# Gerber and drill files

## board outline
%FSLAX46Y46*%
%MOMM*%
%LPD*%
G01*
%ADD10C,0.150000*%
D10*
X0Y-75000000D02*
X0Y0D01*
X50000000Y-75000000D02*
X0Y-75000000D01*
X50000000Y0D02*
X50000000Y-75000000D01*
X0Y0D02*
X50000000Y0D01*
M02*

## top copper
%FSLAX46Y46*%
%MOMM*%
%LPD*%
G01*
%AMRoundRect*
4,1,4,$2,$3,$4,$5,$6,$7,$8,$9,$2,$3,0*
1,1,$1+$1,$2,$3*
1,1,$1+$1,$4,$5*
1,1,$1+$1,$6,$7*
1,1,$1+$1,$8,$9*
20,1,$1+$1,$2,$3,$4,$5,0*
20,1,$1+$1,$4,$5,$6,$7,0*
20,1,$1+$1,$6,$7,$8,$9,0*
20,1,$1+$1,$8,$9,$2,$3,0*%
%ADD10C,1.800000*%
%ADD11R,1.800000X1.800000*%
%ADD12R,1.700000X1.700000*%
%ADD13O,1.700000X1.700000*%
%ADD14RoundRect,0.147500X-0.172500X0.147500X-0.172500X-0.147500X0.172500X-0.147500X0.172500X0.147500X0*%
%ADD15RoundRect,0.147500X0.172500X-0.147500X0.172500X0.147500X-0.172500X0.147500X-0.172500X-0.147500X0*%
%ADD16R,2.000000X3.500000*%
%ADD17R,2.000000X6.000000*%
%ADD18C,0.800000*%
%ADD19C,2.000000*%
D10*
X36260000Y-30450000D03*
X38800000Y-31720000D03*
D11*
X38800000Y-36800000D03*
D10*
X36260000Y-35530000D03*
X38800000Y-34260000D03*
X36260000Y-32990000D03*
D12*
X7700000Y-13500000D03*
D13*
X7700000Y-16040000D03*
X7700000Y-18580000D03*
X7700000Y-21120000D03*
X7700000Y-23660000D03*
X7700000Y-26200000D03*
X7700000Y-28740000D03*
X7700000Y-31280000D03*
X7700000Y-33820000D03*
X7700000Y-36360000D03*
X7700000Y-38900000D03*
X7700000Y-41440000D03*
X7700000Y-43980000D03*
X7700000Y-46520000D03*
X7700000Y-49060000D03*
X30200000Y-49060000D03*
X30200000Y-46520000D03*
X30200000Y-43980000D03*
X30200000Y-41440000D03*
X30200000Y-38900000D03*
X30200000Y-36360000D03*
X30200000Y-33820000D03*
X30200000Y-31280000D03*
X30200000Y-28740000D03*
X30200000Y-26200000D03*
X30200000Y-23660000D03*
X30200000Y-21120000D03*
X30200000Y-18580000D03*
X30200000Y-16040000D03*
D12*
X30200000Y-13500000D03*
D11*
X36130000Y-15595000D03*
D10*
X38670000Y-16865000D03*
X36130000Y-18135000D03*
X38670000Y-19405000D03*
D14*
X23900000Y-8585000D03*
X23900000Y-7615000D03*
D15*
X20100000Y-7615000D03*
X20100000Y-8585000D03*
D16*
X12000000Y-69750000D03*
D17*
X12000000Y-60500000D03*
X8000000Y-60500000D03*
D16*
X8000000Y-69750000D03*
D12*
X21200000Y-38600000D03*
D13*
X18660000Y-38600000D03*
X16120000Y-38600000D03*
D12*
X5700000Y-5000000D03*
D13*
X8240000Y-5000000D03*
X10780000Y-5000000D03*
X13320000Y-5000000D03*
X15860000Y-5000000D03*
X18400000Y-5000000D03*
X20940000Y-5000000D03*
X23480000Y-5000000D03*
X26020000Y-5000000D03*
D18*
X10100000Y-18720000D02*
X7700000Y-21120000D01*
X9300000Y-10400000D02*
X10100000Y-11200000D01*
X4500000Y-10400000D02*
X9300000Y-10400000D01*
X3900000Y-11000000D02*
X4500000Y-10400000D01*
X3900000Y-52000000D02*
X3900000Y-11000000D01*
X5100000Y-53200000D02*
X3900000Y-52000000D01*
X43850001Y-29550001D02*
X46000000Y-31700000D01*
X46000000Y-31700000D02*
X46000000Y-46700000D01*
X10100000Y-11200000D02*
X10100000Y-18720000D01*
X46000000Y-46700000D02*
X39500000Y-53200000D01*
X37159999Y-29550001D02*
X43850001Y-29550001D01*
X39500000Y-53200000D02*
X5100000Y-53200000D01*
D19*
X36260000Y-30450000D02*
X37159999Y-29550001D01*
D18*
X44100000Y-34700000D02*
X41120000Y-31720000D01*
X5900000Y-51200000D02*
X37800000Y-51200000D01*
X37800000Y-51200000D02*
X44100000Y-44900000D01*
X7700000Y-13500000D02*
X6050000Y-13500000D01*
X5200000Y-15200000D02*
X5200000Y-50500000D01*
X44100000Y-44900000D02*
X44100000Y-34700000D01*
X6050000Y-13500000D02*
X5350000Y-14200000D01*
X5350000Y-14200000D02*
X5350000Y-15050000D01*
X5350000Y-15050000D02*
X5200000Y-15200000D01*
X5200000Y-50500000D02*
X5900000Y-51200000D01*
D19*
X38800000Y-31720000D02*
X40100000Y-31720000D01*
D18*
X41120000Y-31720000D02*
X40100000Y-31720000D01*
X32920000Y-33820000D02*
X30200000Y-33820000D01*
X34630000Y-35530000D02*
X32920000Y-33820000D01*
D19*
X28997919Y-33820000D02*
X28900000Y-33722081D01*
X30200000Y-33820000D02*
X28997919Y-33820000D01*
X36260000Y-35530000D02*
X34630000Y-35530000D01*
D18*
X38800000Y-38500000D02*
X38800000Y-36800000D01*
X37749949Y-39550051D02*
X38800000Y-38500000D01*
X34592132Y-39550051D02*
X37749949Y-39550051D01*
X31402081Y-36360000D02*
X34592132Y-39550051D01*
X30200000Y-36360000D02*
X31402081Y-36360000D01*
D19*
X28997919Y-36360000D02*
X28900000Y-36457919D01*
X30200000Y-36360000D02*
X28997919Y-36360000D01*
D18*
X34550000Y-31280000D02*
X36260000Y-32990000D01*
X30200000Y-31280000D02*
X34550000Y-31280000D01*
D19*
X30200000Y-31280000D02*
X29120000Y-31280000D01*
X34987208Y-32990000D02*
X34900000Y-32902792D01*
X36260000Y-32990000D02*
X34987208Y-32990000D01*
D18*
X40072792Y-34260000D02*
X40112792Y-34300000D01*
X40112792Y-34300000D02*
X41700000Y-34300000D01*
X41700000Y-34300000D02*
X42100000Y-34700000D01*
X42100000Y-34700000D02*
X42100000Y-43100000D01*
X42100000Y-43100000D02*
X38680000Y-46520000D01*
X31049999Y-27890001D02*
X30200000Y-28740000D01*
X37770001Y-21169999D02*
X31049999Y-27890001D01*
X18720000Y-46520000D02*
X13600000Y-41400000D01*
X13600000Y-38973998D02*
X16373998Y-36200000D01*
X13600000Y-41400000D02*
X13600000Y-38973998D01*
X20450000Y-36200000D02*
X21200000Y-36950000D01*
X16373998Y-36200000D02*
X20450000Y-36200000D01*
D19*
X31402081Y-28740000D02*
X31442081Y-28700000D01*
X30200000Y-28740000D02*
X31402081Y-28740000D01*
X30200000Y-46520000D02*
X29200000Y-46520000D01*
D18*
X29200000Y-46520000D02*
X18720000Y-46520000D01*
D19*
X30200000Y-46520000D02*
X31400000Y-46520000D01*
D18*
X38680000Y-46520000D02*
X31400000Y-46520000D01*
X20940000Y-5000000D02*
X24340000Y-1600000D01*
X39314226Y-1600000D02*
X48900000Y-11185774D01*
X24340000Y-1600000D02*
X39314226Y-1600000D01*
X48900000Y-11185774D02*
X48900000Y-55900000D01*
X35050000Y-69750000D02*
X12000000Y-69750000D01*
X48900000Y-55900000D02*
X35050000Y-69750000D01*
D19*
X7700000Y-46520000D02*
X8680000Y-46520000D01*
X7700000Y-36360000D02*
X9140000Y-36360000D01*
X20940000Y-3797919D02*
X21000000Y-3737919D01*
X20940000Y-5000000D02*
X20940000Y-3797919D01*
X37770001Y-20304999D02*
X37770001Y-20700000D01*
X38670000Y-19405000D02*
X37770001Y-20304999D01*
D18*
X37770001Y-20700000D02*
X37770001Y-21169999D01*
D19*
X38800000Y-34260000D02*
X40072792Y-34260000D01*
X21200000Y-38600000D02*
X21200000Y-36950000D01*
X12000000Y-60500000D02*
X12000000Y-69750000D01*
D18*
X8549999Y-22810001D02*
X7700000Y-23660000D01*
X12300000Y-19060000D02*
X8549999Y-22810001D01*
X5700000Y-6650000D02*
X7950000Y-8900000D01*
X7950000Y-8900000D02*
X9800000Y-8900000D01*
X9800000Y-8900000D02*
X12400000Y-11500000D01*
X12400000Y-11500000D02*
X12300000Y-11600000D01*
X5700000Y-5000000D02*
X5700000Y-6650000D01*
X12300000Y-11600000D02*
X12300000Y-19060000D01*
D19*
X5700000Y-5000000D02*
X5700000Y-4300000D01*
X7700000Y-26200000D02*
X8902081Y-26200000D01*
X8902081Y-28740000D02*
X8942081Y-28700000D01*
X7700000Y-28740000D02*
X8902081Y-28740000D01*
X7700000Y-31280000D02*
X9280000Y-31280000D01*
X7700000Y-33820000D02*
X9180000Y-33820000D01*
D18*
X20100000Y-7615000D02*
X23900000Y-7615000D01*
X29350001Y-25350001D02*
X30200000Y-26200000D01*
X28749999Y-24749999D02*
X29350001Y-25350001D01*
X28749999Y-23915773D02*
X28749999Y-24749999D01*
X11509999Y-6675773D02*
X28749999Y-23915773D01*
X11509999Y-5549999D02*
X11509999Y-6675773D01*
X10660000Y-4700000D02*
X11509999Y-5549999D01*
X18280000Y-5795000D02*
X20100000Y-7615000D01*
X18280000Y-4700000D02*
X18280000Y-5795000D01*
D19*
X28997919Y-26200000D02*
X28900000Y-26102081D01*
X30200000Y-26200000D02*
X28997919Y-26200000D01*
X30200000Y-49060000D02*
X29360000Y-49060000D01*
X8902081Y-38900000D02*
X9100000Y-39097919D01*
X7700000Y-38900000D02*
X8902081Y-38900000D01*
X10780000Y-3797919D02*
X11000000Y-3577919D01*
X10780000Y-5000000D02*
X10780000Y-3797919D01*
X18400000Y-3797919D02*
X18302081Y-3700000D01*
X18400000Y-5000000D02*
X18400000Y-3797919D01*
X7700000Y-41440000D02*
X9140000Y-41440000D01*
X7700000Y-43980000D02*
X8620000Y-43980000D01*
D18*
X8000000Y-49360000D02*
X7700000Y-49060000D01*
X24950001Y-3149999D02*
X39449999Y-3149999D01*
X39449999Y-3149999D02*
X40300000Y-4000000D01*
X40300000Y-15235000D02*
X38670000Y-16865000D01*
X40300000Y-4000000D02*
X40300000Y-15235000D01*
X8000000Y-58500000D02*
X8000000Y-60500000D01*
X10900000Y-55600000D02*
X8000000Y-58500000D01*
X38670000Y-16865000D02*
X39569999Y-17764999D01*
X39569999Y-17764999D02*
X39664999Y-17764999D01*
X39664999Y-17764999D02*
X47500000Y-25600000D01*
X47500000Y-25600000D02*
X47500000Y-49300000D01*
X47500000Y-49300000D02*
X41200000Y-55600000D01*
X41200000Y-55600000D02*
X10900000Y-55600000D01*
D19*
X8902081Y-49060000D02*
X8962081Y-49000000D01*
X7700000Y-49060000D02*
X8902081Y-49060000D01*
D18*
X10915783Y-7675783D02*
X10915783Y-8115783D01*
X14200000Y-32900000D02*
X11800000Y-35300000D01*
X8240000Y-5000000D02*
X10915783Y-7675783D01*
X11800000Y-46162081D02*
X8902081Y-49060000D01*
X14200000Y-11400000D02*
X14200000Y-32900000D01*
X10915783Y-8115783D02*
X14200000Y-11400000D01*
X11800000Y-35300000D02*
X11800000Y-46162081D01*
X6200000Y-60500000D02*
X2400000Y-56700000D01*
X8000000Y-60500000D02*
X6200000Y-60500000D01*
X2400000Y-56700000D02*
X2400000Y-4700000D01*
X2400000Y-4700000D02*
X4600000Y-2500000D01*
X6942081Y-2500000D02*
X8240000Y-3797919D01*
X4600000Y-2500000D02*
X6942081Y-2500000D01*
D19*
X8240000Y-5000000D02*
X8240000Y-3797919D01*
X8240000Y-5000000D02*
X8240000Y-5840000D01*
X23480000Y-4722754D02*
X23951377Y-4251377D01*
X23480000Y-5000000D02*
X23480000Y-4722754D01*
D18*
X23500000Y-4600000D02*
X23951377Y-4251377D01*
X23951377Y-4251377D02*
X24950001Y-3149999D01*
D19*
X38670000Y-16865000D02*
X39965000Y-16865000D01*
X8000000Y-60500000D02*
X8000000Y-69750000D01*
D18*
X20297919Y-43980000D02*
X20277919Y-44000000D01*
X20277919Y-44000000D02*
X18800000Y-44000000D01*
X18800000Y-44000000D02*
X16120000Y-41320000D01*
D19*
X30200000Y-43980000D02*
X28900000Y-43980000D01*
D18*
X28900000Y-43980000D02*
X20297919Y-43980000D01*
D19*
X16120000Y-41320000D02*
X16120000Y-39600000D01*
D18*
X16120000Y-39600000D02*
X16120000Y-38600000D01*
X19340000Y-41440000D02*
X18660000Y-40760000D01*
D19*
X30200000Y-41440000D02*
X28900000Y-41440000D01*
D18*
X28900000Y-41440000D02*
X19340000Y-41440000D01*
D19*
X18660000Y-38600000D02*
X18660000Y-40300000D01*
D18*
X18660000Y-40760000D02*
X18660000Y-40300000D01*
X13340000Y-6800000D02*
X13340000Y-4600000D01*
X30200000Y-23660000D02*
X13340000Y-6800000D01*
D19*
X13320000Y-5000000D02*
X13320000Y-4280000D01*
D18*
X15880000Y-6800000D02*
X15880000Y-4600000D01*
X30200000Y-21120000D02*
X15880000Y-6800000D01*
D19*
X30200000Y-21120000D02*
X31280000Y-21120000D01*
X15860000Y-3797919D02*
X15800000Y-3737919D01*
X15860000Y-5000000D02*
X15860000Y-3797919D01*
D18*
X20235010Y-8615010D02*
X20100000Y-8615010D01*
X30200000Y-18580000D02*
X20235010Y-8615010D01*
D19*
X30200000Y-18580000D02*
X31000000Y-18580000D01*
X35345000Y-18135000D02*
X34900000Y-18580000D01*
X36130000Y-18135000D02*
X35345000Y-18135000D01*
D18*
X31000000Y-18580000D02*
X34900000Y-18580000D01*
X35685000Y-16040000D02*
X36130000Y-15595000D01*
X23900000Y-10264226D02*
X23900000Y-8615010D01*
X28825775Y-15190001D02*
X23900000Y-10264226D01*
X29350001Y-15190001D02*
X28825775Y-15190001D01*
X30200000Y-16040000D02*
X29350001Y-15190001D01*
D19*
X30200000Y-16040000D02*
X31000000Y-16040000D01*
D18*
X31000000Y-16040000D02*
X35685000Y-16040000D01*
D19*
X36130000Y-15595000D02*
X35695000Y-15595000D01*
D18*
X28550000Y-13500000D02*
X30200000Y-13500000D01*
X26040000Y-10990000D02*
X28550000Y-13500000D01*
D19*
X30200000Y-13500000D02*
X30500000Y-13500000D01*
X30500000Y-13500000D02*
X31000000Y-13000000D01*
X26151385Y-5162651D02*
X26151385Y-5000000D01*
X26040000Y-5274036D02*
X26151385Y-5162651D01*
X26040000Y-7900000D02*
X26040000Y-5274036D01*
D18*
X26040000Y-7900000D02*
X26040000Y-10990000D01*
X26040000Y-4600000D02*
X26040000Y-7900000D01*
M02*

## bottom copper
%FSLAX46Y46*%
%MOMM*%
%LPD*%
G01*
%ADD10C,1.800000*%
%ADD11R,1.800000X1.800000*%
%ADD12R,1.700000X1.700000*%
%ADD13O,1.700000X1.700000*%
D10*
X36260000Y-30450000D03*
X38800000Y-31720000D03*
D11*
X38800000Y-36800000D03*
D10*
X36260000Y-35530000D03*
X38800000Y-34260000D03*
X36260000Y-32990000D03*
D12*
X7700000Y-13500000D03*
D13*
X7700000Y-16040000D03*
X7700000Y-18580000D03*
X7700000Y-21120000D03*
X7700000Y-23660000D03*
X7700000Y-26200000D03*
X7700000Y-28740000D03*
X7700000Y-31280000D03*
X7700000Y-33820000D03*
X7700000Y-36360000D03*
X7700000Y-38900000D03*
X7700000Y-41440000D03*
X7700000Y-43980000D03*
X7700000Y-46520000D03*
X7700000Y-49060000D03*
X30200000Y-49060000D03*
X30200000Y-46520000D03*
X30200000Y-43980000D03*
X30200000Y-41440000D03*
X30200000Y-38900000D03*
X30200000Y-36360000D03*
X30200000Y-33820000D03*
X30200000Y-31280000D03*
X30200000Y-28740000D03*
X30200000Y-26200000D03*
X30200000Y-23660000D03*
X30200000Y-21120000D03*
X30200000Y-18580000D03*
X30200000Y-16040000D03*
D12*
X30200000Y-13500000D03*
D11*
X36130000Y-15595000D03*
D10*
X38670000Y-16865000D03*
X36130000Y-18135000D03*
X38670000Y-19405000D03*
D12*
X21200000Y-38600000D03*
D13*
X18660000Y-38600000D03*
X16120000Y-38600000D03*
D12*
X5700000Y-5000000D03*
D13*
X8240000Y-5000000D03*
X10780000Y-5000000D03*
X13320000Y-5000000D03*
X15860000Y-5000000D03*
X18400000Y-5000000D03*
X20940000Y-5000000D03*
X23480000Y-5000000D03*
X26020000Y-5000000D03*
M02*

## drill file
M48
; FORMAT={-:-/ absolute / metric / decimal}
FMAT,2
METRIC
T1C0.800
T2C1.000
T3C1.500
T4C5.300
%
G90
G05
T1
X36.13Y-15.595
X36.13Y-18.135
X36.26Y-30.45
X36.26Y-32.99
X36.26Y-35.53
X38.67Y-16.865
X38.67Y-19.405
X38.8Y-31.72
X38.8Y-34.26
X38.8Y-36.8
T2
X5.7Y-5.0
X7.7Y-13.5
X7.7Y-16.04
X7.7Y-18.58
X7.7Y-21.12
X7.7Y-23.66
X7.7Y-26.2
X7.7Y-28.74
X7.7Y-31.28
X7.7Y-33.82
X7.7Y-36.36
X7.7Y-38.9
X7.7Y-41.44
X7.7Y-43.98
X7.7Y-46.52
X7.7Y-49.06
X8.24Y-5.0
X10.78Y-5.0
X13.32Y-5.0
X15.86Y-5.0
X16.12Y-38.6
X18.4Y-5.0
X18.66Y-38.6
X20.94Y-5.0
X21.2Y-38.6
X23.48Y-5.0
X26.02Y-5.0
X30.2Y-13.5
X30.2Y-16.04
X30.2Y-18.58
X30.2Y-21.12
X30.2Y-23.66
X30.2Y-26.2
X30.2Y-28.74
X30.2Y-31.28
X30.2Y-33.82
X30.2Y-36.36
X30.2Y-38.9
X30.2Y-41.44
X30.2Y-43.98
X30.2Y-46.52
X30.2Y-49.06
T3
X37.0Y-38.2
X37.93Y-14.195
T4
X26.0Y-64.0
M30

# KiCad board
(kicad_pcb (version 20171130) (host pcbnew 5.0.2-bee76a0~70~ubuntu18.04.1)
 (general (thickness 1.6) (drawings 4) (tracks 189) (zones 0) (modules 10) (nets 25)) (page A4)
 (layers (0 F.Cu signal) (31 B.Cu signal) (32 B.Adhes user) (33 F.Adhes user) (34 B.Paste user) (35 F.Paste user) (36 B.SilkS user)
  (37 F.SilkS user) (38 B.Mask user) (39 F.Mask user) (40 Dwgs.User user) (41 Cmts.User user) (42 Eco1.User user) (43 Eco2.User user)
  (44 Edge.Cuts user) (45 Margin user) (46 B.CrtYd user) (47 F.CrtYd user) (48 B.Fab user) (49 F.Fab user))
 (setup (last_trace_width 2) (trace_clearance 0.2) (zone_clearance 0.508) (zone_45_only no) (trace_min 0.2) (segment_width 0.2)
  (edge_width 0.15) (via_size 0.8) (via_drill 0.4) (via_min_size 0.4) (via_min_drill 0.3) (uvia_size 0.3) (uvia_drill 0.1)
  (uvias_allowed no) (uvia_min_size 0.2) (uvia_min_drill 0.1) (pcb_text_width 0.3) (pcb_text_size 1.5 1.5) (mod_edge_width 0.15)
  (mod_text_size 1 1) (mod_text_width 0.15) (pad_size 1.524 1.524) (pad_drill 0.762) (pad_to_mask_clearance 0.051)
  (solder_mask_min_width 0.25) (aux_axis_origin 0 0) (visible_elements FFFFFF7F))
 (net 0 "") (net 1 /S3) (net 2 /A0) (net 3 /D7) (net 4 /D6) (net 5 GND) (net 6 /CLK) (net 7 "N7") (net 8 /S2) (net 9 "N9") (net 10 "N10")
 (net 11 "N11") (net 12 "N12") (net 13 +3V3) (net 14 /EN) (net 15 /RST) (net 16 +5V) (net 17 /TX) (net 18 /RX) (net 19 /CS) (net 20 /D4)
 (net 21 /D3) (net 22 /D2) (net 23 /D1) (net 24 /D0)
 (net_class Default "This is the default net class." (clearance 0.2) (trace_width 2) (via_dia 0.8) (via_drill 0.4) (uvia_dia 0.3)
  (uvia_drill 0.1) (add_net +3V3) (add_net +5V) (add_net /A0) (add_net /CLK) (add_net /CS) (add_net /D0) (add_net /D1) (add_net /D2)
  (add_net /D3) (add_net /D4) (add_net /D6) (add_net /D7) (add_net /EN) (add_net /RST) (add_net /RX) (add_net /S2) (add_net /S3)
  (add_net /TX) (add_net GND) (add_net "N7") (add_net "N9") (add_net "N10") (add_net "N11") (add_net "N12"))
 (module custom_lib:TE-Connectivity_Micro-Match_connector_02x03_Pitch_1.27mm (layer F.Cu) (at 38.8 36.8 180)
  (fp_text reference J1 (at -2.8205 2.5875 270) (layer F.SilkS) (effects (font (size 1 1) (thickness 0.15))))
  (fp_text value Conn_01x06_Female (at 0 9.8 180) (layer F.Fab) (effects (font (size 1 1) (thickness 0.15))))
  (pad 6 thru_hole circle (at 2.54 6.35 180) (size 1.8 1.8) (drill 0.8001) (layers *.Cu *.Mask) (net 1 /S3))
  (pad 5 thru_hole circle (at 0 5.08 180) (size 1.8 1.8) (drill 0.8001) (layers *.Cu *.Mask) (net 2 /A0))
  (pad 1 thru_hole rect (at 0 0 180) (size 1.8 1.8) (drill 0.8001) (layers *.Cu *.Mask) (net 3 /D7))
  (pad 2 thru_hole circle (at 2.54 1.27 180) (size 1.8 1.8) (drill 0.8001) (layers *.Cu *.Mask) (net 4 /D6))
  (pad 3 thru_hole circle (at 0 2.54 180) (size 1.8 1.8) (drill 0.8001) (layers *.Cu *.Mask) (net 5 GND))
  (pad 4 thru_hole circle (at 2.54 3.81 180) (size 1.8 1.8) (drill 0.8001) (layers *.Cu *.Mask) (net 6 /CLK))
  (pad "" np_thru_hole circle (at 1.8 -1.4 180) (size 1.5001 1.5001) (drill 1.5001) (layers *.Cu *.Mask)))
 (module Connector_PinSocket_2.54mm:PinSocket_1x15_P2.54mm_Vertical (layer F.Cu) (at 7.7 13.5)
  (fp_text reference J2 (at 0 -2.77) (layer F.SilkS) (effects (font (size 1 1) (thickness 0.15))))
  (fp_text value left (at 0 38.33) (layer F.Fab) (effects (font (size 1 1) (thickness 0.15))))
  (pad 1 thru_hole rect (at 0 0) (size 1.7 1.7) (drill 1) (layers *.Cu *.Mask) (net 2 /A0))
  (pad 2 thru_hole oval (at 0 2.54) (size 1.7 1.7) (drill 1) (layers *.Cu *.Mask) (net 5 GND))
  (pad 3 thru_hole oval (at 0 5.08) (size 1.7 1.7) (drill 1) (layers *.Cu *.Mask) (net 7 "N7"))
  (pad 4 thru_hole oval (at 0 7.62) (size 1.7 1.7) (drill 1) (layers *.Cu *.Mask) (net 1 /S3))
  (pad 5 thru_hole oval (at 0 10.16) (size 1.7 1.7) (drill 1) (layers *.Cu *.Mask) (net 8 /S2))
  (pad 6 thru_hole oval (at 0 12.7) (size 1.7 1.7) (drill 1) (layers *.Cu *.Mask) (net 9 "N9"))
  (pad 7 thru_hole oval (at 0 15.24) (size 1.7 1.7) (drill 1) (layers *.Cu *.Mask) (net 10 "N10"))
  (pad 8 thru_hole oval (at 0 17.78) (size 1.7 1.7) (drill 1) (layers *.Cu *.Mask) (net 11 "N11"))
  (pad 9 thru_hole oval (at 0 20.32) (size 1.7 1.7) (drill 1) (layers *.Cu *.Mask) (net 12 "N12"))
  (pad 10 thru_hole oval (at 0 22.86) (size 1.7 1.7) (drill 1) (layers *.Cu *.Mask) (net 5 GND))
  (pad 11 thru_hole oval (at 0 25.4) (size 1.7 1.7) (drill 1) (layers *.Cu *.Mask) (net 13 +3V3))
  (pad 12 thru_hole oval (at 0 27.94) (size 1.7 1.7) (drill 1) (layers *.Cu *.Mask) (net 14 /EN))
  (pad 13 thru_hole oval (at 0 30.48) (size 1.7 1.7) (drill 1) (layers *.Cu *.Mask) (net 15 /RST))
  (pad 14 thru_hole oval (at 0 33.02) (size 1.7 1.7) (drill 1) (layers *.Cu *.Mask) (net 5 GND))
  (pad 15 thru_hole oval (at 0 35.56) (size 1.7 1.7) (drill 1) (layers *.Cu *.Mask) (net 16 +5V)))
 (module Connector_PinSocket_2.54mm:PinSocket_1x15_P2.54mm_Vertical (layer F.Cu) (at 30.2 13.5)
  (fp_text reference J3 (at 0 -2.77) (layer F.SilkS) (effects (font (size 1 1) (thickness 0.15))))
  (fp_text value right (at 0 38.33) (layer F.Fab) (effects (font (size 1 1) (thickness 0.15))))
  (pad 15 thru_hole oval (at 0 35.56) (size 1.7 1.7) (drill 1) (layers *.Cu *.Mask) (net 13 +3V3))
  (pad 14 thru_hole oval (at 0 33.02) (size 1.7 1.7) (drill 1) (layers *.Cu *.Mask) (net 5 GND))
  (pad 13 thru_hole oval (at 0 30.48) (size 1.7 1.7) (drill 1) (layers *.Cu *.Mask) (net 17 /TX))
  (pad 12 thru_hole oval (at 0 27.94) (size 1.7 1.7) (drill 1) (layers *.Cu *.Mask) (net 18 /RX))
  (pad 11 thru_hole oval (at 0 25.4) (size 1.7 1.7) (drill 1) (layers *.Cu *.Mask) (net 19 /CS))
  (pad 10 thru_hole oval (at 0 22.86) (size 1.7 1.7) (drill 1) (layers *.Cu *.Mask) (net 3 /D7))
  (pad 9 thru_hole oval (at 0 20.32) (size 1.7 1.7) (drill 1) (layers *.Cu *.Mask) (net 4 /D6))
  (pad 8 thru_hole oval (at 0 17.78) (size 1.7 1.7) (drill 1) (layers *.Cu *.Mask) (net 6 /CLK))
  (pad 7 thru_hole oval (at 0 15.24) (size 1.7 1.7) (drill 1) (layers *.Cu *.Mask) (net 5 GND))
  (pad 6 thru_hole oval (at 0 12.7) (size 1.7 1.7) (drill 1) (layers *.Cu *.Mask) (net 13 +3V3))
  (pad 5 thru_hole oval (at 0 10.16) (size 1.7 1.7) (drill 1) (layers *.Cu *.Mask) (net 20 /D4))
  (pad 4 thru_hole oval (at 0 7.62) (size 1.7 1.7) (drill 1) (layers *.Cu *.Mask) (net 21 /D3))
  (pad 3 thru_hole oval (at 0 5.08) (size 1.7 1.7) (drill 1) (layers *.Cu *.Mask) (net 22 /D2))
  (pad 2 thru_hole oval (at 0 2.54) (size 1.7 1.7) (drill 1) (layers *.Cu *.Mask) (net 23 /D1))
  (pad 1 thru_hole rect (at 0 0) (size 1.7 1.7) (drill 1) (layers *.Cu *.Mask) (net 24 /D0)))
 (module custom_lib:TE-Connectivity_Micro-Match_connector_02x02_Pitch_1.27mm (layer F.Cu) (at 37.4 17.5)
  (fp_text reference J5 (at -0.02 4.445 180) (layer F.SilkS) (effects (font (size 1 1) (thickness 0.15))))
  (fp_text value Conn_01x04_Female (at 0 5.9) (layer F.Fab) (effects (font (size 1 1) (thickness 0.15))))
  (pad 1 thru_hole rect (at -1.27 -1.905) (size 1.8 1.8) (drill 0.8001) (layers *.Cu *.Mask) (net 23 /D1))
  (pad 2 thru_hole circle (at 1.27 -0.635) (size 1.8 1.8) (drill 0.8001) (layers *.Cu *.Mask) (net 16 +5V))
  (pad 3 thru_hole circle (at -1.27 0.635) (size 1.8 1.8) (drill 0.8001) (layers *.Cu *.Mask) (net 22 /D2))
  (pad 4 thru_hole circle (at 1.27 1.905) (size 1.8 1.8) (drill 0.8001) (layers *.Cu *.Mask) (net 5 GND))
  (pad "" np_thru_hole circle (at 0.53 -3.305) (size 1.5001 1.5001) (drill 1.5001) (layers *.Cu *.Mask)))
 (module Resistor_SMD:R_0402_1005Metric (layer F.Cu) (at 23.9 8.1 270)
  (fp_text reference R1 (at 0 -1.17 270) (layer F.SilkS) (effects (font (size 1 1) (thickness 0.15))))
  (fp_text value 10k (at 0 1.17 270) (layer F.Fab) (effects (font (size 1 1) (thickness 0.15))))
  (pad 2 smd roundrect (at 0.485 0 270) (size 0.59 0.64) (layers F.Cu F.Paste F.Mask) (roundrect_rratio 0.25) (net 23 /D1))
  (pad 1 smd roundrect (at -0.485 0 270) (size 0.59 0.64) (layers F.Cu F.Paste F.Mask) (roundrect_rratio 0.25) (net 13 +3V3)))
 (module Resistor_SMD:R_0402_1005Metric (layer F.Cu) (at 20.1 8.1 90)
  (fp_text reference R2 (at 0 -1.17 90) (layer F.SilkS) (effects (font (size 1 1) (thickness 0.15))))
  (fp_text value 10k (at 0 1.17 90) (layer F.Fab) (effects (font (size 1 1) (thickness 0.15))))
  (pad 2 smd roundrect (at 0.485 0 90) (size 0.59 0.64) (layers F.Cu F.Paste F.Mask) (roundrect_rratio 0.25) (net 13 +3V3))
  (pad 1 smd roundrect (at -0.485 0 90) (size 0.59 0.64) (layers F.Cu F.Paste F.Mask) (roundrect_rratio 0.25) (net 22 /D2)))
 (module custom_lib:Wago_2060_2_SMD (layer F.Cu) (at 10 64.5)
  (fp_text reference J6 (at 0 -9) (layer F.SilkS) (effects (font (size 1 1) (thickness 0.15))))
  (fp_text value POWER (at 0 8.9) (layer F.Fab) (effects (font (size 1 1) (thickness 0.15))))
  (pad 2 smd rect (at 2 5.25) (size 2 3.5) (layers F.Cu F.Paste F.Mask) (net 5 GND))
  (pad 2 smd rect (at 2 -4) (size 2 6) (layers F.Cu F.Paste F.Mask) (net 5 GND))
  (pad 1 smd rect (at -2 -4) (size 2 6) (layers F.Cu F.Paste F.Mask) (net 16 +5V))
  (pad 1 smd rect (at -2 5.25) (size 2 3.5) (layers F.Cu F.Paste F.Mask) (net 16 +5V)))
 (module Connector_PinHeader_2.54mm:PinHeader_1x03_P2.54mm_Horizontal (layer F.Cu) (at 21.2 38.6 270)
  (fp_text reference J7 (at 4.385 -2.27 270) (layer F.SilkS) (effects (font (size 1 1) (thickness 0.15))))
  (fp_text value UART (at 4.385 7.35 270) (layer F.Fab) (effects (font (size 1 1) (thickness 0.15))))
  (pad 1 thru_hole rect (at 0 0 270) (size 1.7 1.7) (drill 1) (layers *.Cu *.Mask) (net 5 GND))
  (pad 2 thru_hole oval (at 0 2.54 270) (size 1.7 1.7) (drill 1) (layers *.Cu *.Mask) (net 18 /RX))
  (pad 3 thru_hole oval (at 0 5.08 270) (size 1.7 1.7) (drill 1) (layers *.Cu *.Mask) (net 17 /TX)))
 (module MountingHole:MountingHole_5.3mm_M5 (layer F.Cu) (at 26 64)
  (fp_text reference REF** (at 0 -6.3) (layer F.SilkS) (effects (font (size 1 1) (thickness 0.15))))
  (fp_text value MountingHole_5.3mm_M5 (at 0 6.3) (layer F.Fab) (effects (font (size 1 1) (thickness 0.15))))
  (pad 1 np_thru_hole circle (at 0 0) (size 5.3 5.3) (drill 5.3) (layers *.Cu *.Mask)))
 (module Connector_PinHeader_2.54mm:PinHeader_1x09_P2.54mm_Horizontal (layer F.Cu) (at 5.7 5 90)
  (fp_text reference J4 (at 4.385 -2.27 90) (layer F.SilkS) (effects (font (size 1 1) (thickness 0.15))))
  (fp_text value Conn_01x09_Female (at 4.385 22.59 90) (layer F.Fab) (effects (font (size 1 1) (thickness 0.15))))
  (pad 1 thru_hole rect (at 0 0 90) (size 1.7 1.7) (drill 1) (layers *.Cu *.Mask) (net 8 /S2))
  (pad 2 thru_hole oval (at 0 2.54 90) (size 1.7 1.7) (drill 1) (layers *.Cu *.Mask) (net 16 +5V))
  (pad 3 thru_hole oval (at 0 5.08 90) (size 1.7 1.7) (drill 1) (layers *.Cu *.Mask) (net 13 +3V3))
  (pad 4 thru_hole oval (at 0 7.62 90) (size 1.7 1.7) (drill 1) (layers *.Cu *.Mask) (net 20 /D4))
  (pad 5 thru_hole oval (at 0 10.16 90) (size 1.7 1.7) (drill 1) (layers *.Cu *.Mask) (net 21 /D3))
  (pad 6 thru_hole oval (at 0 12.7 90) (size 1.7 1.7) (drill 1) (layers *.Cu *.Mask) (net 13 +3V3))
  (pad 7 thru_hole oval (at 0 15.24 90) (size 1.7 1.7) (drill 1) (layers *.Cu *.Mask) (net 5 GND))
  (pad 8 thru_hole oval (at 0 17.78 90) (size 1.7 1.7) (drill 1) (layers *.Cu *.Mask) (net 16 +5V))
  (pad 9 thru_hole oval (at 0 20.32 90) (size 1.7 1.7) (drill 1) (layers *.Cu *.Mask) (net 24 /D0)))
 (gr_line (start 0 75) (end 0 0) (layer Edge.Cuts) (width 0.15))
 (gr_line (start 50 75) (end 0 75) (layer Edge.Cuts) (width 0.15))
 (gr_line (start 50 0) (end 50 75) (layer Edge.Cuts) (width 0.15))
 (gr_line (start 0 0) (end 50 0) (layer Edge.Cuts) (width 0.15))
 (segment (start 10.1 18.72) (end 7.7 21.12) (width 0.8) (layer F.Cu) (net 1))
 (segment (start 9.3 10.4) (end 10.1 11.2) (width 0.8) (layer F.Cu) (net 1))
 (segment (start 4.5 10.4) (end 9.3 10.4) (width 0.8) (layer F.Cu) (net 1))
 (segment (start 3.9 11) (end 4.5 10.4) (width 0.8) (layer F.Cu) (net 1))
 (segment (start 3.9 52) (end 3.9 11) (width 0.8) (layer F.Cu) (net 1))
 (segment (start 5.1 53.2) (end 3.9 52) (width 0.8) (layer F.Cu) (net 1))
 (segment (start 43.850001 29.550001) (end 46 31.7) (width 0.8) (layer F.Cu) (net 1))
 (segment (start 46 31.7) (end 46 46.7) (width 0.8) (layer F.Cu) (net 1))
 (segment (start 10.1 11.2) (end 10.1 18.72) (width 0.8) (layer F.Cu) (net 1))
 (segment (start 46 46.7) (end 39.5 53.2) (width 0.8) (layer F.Cu) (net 1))
 (segment (start 37.159999 29.550001) (end 43.850001 29.550001) (width 0.8) (layer F.Cu) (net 1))
 (segment (start 39.5 53.2) (end 5.1 53.2) (width 0.8) (layer F.Cu) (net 1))
 (segment (start 36.26 30.45) (end 37.159999 29.550001) (width 2) (layer F.Cu) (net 1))
 (segment (start 44.1 34.7) (end 41.12 31.72) (width 0.8) (layer F.Cu) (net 2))
 (segment (start 5.9 51.2) (end 37.8 51.2) (width 0.8) (layer F.Cu) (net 2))
 (segment (start 37.8 51.2) (end 44.1 44.9) (width 0.8) (layer F.Cu) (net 2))
 (segment (start 7.7 13.5) (end 6.05 13.5) (width 0.8) (layer F.Cu) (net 2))
 (segment (start 5.2 15.2) (end 5.2 50.5) (width 0.8) (layer F.Cu) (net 2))
 (segment (start 44.1 44.9) (end 44.1 34.7) (width 0.8) (layer F.Cu) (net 2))
 (segment (start 6.05 13.5) (end 5.35 14.2) (width 0.8) (layer F.Cu) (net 2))
 (segment (start 5.35 14.2) (end 5.35 15.05) (width 0.8) (layer F.Cu) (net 2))
 (segment (start 5.35 15.05) (end 5.2 15.2) (width 0.8) (layer F.Cu) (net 2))
 (segment (start 5.2 50.5) (end 5.9 51.2) (width 0.8) (layer F.Cu) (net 2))
 (segment (start 38.8 31.72) (end 40.1 31.72) (width 2) (layer F.Cu) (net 2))
 (segment (start 41.12 31.72) (end 40.1 31.72) (width 0.8) (layer F.Cu) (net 2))
 (segment (start 32.92 33.82) (end 30.2 33.82) (width 0.8) (layer F.Cu) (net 4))
 (segment (start 34.63 35.53) (end 32.92 33.82) (width 0.8) (layer F.Cu) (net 4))
 (segment (start 28.997919 33.82) (end 28.9 33.722081) (width 2) (layer F.Cu) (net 4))
 (segment (start 30.2 33.82) (end 28.997919 33.82) (width 2) (layer F.Cu) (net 4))
 (segment (start 36.26 35.53) (end 34.63 35.53) (width 2) (layer F.Cu) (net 4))
 (segment (start 38.8 38.5) (end 38.8 36.8) (width 0.8) (layer F.Cu) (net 3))
 (segment (start 37.749949 39.550051) (end 38.8 38.5) (width 0.8) (layer F.Cu) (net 3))
 (segment (start 34.592132 39.550051) (end 37.749949 39.550051) (width 0.8) (layer F.Cu) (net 3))
 (segment (start 31.402081 36.36) (end 34.592132 39.550051) (width 0.8) (layer F.Cu) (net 3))
 (segment (start 30.2 36.36) (end 31.402081 36.36) (width 0.8) (layer F.Cu) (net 3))
 (segment (start 28.997919 36.36) (end 28.9 36.457919) (width 2) (layer F.Cu) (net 3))
 (segment (start 30.2 36.36) (end 28.997919 36.36) (width 2) (layer F.Cu) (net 3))
 (segment (start 34.55 31.28) (end 36.26 32.99) (width 0.8) (layer F.Cu) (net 6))
 (segment (start 30.2 31.28) (end 34.55 31.28) (width 0.8) (layer F.Cu) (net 6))
 (segment (start 30.2 31.28) (end 29.12 31.28) (width 2) (layer F.Cu) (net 6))
 (segment (start 34.987208 32.99) (end 34.9 32.902792) (width 2) (layer F.Cu) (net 6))
 (segment (start 36.26 32.99) (end 34.987208 32.99) (width 2) (layer F.Cu) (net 6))
 (segment (start 40.072792 34.26) (end 40.112792 34.3) (width 0.8) (layer F.Cu) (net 5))
 (segment (start 40.112792 34.3) (end 41.7 34.3) (width 0.8) (layer F.Cu) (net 5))
 (segment (start 41.7 34.3) (end 42.1 34.7) (width 0.8) (layer F.Cu) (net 5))
 (segment (start 42.1 34.7) (end 42.1 43.1) (width 0.8) (layer F.Cu) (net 5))
 (segment (start 42.1 43.1) (end 38.68 46.52) (width 0.8) (layer F.Cu) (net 5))
 (segment (start 31.049999 27.890001) (end 30.2 28.74) (width 0.8) (layer F.Cu) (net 5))
 (segment (start 37.770001 21.169999) (end 31.049999 27.890001) (width 0.8) (layer F.Cu) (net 5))
 (segment (start 18.72 46.52) (end 13.6 41.4) (width 0.8) (layer F.Cu) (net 5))
 (segment (start 13.6 38.973998) (end 16.373998 36.2) (width 0.8) (layer F.Cu) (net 5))
 (segment (start 13.6 41.4) (end 13.6 38.973998) (width 0.8) (layer F.Cu) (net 5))
 (segment (start 20.45 36.2) (end 21.2 36.95) (width 0.8) (layer F.Cu) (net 5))
 (segment (start 16.373998 36.2) (end 20.45 36.2) (width 0.8) (layer F.Cu) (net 5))
 (segment (start 31.402081 28.74) (end 31.442081 28.7) (width 2) (layer F.Cu) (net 5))
 (segment (start 30.2 28.74) (end 31.402081 28.74) (width 2) (layer F.Cu) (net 5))
 (segment (start 30.2 46.52) (end 29.2 46.52) (width 2) (layer F.Cu) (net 5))
 (segment (start 29.2 46.52) (end 18.72 46.52) (width 0.8) (layer F.Cu) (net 5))
 (segment (start 30.2 46.52) (end 31.4 46.52) (width 2) (layer F.Cu) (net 5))
 (segment (start 38.68 46.52) (end 31.4 46.52) (width 0.8) (layer F.Cu) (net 5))
 (segment (start 20.94 5) (end 24.34 1.6) (width 0.8) (layer F.Cu) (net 5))
 (segment (start 39.314226 1.6) (end 48.9 11.185774) (width 0.8) (layer F.Cu) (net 5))
 (segment (start 24.34 1.6) (end 39.314226 1.6) (width 0.8) (layer F.Cu) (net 5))
 (segment (start 48.9 11.185774) (end 48.9 55.9) (width 0.8) (layer F.Cu) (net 5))
 (segment (start 35.05 69.75) (end 12 69.75) (width 0.8) (layer F.Cu) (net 5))
 (segment (start 48.9 55.9) (end 35.05 69.75) (width 0.8) (layer F.Cu) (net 5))
 (segment (start 7.7 46.52) (end 8.68 46.52) (width 2) (layer F.Cu) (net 5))
 (segment (start 7.7 36.36) (end 9.14 36.36) (width 2) (layer F.Cu) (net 5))
 (segment (start 20.94 3.797919) (end 21 3.737919) (width 2) (layer F.Cu) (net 5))
 (segment (start 20.94 5) (end 20.94 3.797919) (width 2) (layer F.Cu) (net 5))
 (segment (start 37.770001 20.304999) (end 37.770001 20.7) (width 2) (layer F.Cu) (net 5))
 (segment (start 38.67 19.405) (end 37.770001 20.304999) (width 2) (layer F.Cu) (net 5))
 (segment (start 37.770001 20.7) (end 37.770001 21.169999) (width 0.8) (layer F.Cu) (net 5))
 (segment (start 38.8 34.26) (end 40.072792 34.26) (width 2) (layer F.Cu) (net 5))
 (segment (start 21.2 38.6) (end 21.2 36.95) (width 2) (layer F.Cu) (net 5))
 (segment (start 12 60.5) (end 12 69.75) (width 2) (layer F.Cu) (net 5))
 (segment (start 8.549999 22.810001) (end 7.7 23.66) (width 0.8) (layer F.Cu) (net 8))
 (segment (start 12.3 19.06) (end 8.549999 22.810001) (width 0.8) (layer F.Cu) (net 8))
 (segment (start 5.7 6.65) (end 7.95 8.9) (width 0.8) (layer F.Cu) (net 8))
 (segment (start 7.95 8.9) (end 9.8 8.9) (width 0.8) (layer F.Cu) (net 8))
 (segment (start 9.8 8.9) (end 12.4 11.5) (width 0.8) (layer F.Cu) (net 8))
 (segment (start 12.4 11.5) (end 12.3 11.6) (width 0.8) (layer F.Cu) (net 8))
 (segment (start 5.7 5) (end 5.7 6.65) (width 0.8) (layer F.Cu) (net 8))
 (segment (start 12.3 11.6) (end 12.3 19.06) (width 0.8) (layer F.Cu) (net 8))
 (segment (start 5.7 5) (end 5.7 4.3) (width 2) (layer F.Cu) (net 8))
 (segment (start 7.7 26.2) (end 8.902081 26.2) (width 2) (layer F.Cu) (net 9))
 (segment (start 8.902081 28.74) (end 8.942081 28.7) (width 2) (layer F.Cu) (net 10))
 (segment (start 7.7 28.74) (end 8.902081 28.74) (width 2) (layer F.Cu) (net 10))
 (segment (start 7.7 31.28) (end 9.28 31.28) (width 2) (layer F.Cu) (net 11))
 (segment (start 7.7 33.82) (end 9.18 33.82) (width 2) (layer F.Cu) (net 12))
 (segment (start 20.1 7.615) (end 23.9 7.615) (width 0.8) (layer F.Cu) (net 13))
 (segment (start 29.350001 25.350001) (end 30.2 26.2) (width 0.8) (layer F.Cu) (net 13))
 (segment (start 28.749999 24.749999) (end 29.350001 25.350001) (width 0.8) (layer F.Cu) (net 13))
 (segment (start 28.749999 23.915773) (end 28.749999 24.749999) (width 0.8) (layer F.Cu) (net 13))
 (segment (start 11.509999 6.675773) (end 28.749999 23.915773) (width 0.8) (layer F.Cu) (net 13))
 (segment (start 11.509999 5.549999) (end 11.509999 6.675773) (width 0.8) (layer F.Cu) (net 13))
 (segment (start 10.66 4.7) (end 11.509999 5.549999) (width 0.8) (layer F.Cu) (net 13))
 (segment (start 18.28 5.795) (end 20.1 7.615) (width 0.8) (layer F.Cu) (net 13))
 (segment (start 18.28 4.7) (end 18.28 5.795) (width 0.8) (layer F.Cu) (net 13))
 (segment (start 28.997919 26.2) (end 28.9 26.102081) (width 2) (layer F.Cu) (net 13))
 (segment (start 30.2 26.2) (end 28.997919 26.2) (width 2) (layer F.Cu) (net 13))
 (segment (start 30.2 49.06) (end 29.36 49.06) (width 2) (layer F.Cu) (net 13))
 (segment (start 8.902081 38.9) (end 9.1 39.097919) (width 2) (layer F.Cu) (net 13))
 (segment (start 7.7 38.9) (end 8.902081 38.9) (width 2) (layer F.Cu) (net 13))
 (segment (start 10.78 3.797919) (end 11 3.577919) (width 2) (layer F.Cu) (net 13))
 (segment (start 10.78 5) (end 10.78 3.797919) (width 2) (layer F.Cu) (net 13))
 (segment (start 18.4 3.797919) (end 18.302081 3.7) (width 2) (layer F.Cu) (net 13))
 (segment (start 18.4 5) (end 18.4 3.797919) (width 2) (layer F.Cu) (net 13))
 (segment (start 7.7 41.44) (end 9.14 41.44) (width 2) (layer F.Cu) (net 14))
 (segment (start 7.7 43.98) (end 8.62 43.98) (width 2) (layer F.Cu) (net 15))
 (segment (start 8 49.36) (end 7.7 49.06) (width 0.8) (layer F.Cu) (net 16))
 (segment (start 24.950001 3.149999) (end 39.449999 3.149999) (width 0.8) (layer F.Cu) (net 16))
 (segment (start 39.449999 3.149999) (end 40.3 4) (width 0.8) (layer F.Cu) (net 16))
 (segment (start 40.3 15.235) (end 38.67 16.865) (width 0.8) (layer F.Cu) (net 16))
 (segment (start 40.3 4) (end 40.3 15.235) (width 0.8) (layer F.Cu) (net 16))
 (segment (start 8 58.5) (end 8 60.5) (width 0.8) (layer F.Cu) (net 16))
 (segment (start 10.9 55.6) (end 8 58.5) (width 0.8) (layer F.Cu) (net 16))
 (segment (start 38.67 16.865) (end 39.569999 17.764999) (width 0.8) (layer F.Cu) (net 16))
 (segment (start 39.569999 17.764999) (end 39.664999 17.764999) (width 0.8) (layer F.Cu) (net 16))
 (segment (start 39.664999 17.764999) (end 47.5 25.6) (width 0.8) (layer F.Cu) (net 16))
 (segment (start 47.5 25.6) (end 47.5 49.3) (width 0.8) (layer F.Cu) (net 16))
 (segment (start 47.5 49.3) (end 41.2 55.6) (width 0.8) (layer F.Cu) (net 16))
 (segment (start 41.2 55.6) (end 10.9 55.6) (width 0.8) (layer F.Cu) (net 16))
 (segment (start 8.902081 49.06) (end 8.962081 49) (width 2) (layer F.Cu) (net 16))
 (segment (start 7.7 49.06) (end 8.902081 49.06) (width 2) (layer F.Cu) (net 16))
 (segment (start 10.915783 7.675783) (end 10.915783 8.115783) (width 0.8) (layer F.Cu) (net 16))
 (segment (start 14.2 32.9) (end 11.8 35.3) (width 0.8) (layer F.Cu) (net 16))
 (segment (start 8.24 5) (end 10.915783 7.675783) (width 0.8) (layer F.Cu) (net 16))
 (segment (start 11.8 46.162081) (end 8.902081 49.06) (width 0.8) (layer F.Cu) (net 16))
 (segment (start 14.2 11.4) (end 14.2 32.9) (width 0.8) (layer F.Cu) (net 16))
 (segment (start 10.915783 8.115783) (end 14.2 11.4) (width 0.8) (layer F.Cu) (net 16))
 (segment (start 11.8 35.3) (end 11.8 46.162081) (width 0.8) (layer F.Cu) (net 16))
 (segment (start 6.2 60.5) (end 2.4 56.7) (width 0.8) (layer F.Cu) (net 16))
 (segment (start 8 60.5) (end 6.2 60.5) (width 0.8) (layer F.Cu) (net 16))
 (segment (start 2.4 56.7) (end 2.4 4.7) (width 0.8) (layer F.Cu) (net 16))
 (segment (start 2.4 4.7) (end 4.6 2.5) (width 0.8) (layer F.Cu) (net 16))
 (segment (start 6.942081 2.5) (end 8.24 3.797919) (width 0.8) (layer F.Cu) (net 16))
 (segment (start 4.6 2.5) (end 6.942081 2.5) (width 0.8) (layer F.Cu) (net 16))
 (segment (start 8.24 5) (end 8.24 3.797919) (width 2) (layer F.Cu) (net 16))
 (segment (start 8.24 5) (end 8.24 5.84) (width 2) (layer F.Cu) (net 16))
 (segment (start 23.48 4.722754) (end 23.951377 4.251377) (width 2) (layer F.Cu) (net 16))
 (segment (start 23.48 5) (end 23.48 4.722754) (width 2) (layer F.Cu) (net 16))
 (segment (start 23.5 4.6) (end 23.951377 4.251377) (width 0.8) (layer F.Cu) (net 16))
 (segment (start 23.951377 4.251377) (end 24.950001 3.149999) (width 0.8) (layer F.Cu) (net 16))
 (segment (start 38.67 16.865) (end 39.965 16.865) (width 2) (layer F.Cu) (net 16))
 (segment (start 8 60.5) (end 8 69.75) (width 2) (layer F.Cu) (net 16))
 (segment (start 20.297919 43.98) (end 20.277919 44) (width 0.8) (layer F.Cu) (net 17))
 (segment (start 20.277919 44) (end 18.8 44) (width 0.8) (layer F.Cu) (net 17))
 (segment (start 18.8 44) (end 16.12 41.32) (width 0.8) (layer F.Cu) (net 17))
 (segment (start 30.2 43.98) (end 28.9 43.98) (width 2) (layer F.Cu) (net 17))
 (segment (start 28.9 43.98) (end 20.297919 43.98) (width 0.8) (layer F.Cu) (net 17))
 (segment (start 16.12 41.32) (end 16.12 39.6) (width 2) (layer F.Cu) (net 17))
 (segment (start 16.12 39.6) (end 16.12 38.6) (width 0.8) (layer F.Cu) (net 17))
 (segment (start 19.34 41.44) (end 18.66 40.76) (width 0.8) (layer F.Cu) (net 18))
 (segment (start 30.2 41.44) (end 28.9 41.44) (width 2) (layer F.Cu) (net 18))
 (segment (start 28.9 41.44) (end 19.34 41.44) (width 0.8) (layer F.Cu) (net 18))
 (segment (start 18.66 38.6) (end 18.66 40.3) (width 2) (layer F.Cu) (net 18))
 (segment (start 18.66 40.76) (end 18.66 40.3) (width 0.8) (layer F.Cu) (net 18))
 (segment (start 13.34 6.8) (end 13.34 4.6) (width 0.8) (layer F.Cu) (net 20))
 (segment (start 30.2 23.66) (end 13.34 6.8) (width 0.8) (layer F.Cu) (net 20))
 (segment (start 13.32 5) (end 13.32 4.28) (width 2) (layer F.Cu) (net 20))
 (segment (start 15.88 6.8) (end 15.88 4.6) (width 0.8) (layer F.Cu) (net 21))
 (segment (start 30.2 21.12) (end 15.88 6.8) (width 0.8) (layer F.Cu) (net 21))
 (segment (start 30.2 21.12) (end 31.28 21.12) (width 2) (layer F.Cu) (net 21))
 (segment (start 15.86 3.797919) (end 15.8 3.737919) (width 2) (layer F.Cu) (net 21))
 (segment (start 15.86 5) (end 15.86 3.797919) (width 2) (layer F.Cu) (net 21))
 (segment (start 20.23501 8.61501) (end 20.1 8.61501) (width 0.8) (layer F.Cu) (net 22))
 (segment (start 30.2 18.58) (end 20.23501 8.61501) (width 0.8) (layer F.Cu) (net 22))
 (segment (start 30.2 18.58) (end 31 18.58) (width 2) (layer F.Cu) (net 22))
 (segment (start 35.345 18.135) (end 34.9 18.58) (width 2) (layer F.Cu) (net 22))
 (segment (start 36.13 18.135) (end 35.345 18.135) (width 2) (layer F.Cu) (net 22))
 (segment (start 31 18.58) (end 34.9 18.58) (width 0.8) (layer F.Cu) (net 22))
 (segment (start 35.685 16.04) (end 36.13 15.595) (width 0.8) (layer F.Cu) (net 23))
 (segment (start 23.9 10.264226) (end 23.9 8.61501) (width 0.8) (layer F.Cu) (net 23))
 (segment (start 28.825775 15.190001) (end 23.9 10.264226) (width 0.8) (layer F.Cu) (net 23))
 (segment (start 29.350001 15.190001) (end 28.825775 15.190001) (width 0.8) (layer F.Cu) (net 23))
 (segment (start 30.2 16.04) (end 29.350001 15.190001) (width 0.8) (layer F.Cu) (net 23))
 (segment (start 30.2 16.04) (end 31 16.04) (width 2) (layer F.Cu) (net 23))
 (segment (start 31 16.04) (end 35.685 16.04) (width 0.8) (layer F.Cu) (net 23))
 (segment (start 36.13 15.595) (end 35.695 15.595) (width 2) (layer F.Cu) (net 23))
 (segment (start 28.55 13.5) (end 30.2 13.5) (width 0.8) (layer F.Cu) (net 24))
 (segment (start 26.04 10.99) (end 28.55 13.5) (width 0.8) (layer F.Cu) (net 24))
 (segment (start 30.2 13.5) (end 30.5 13.5) (width 2) (layer F.Cu) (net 24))
 (segment (start 30.5 13.5) (end 31 13) (width 2) (layer F.Cu) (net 24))
 (segment (start 26.151385 5.162651) (end 26.151385 5) (width 2) (layer F.Cu) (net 24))
 (segment (start 26.04 5.274036) (end 26.151385 5.162651) (width 2) (layer F.Cu) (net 24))
 (segment (start 26.04 7.9) (end 26.04 5.274036) (width 2) (layer F.Cu) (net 24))
 (segment (start 26.04 7.9) (end 26.04 10.99) (width 0.8) (layer F.Cu) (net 24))
 (segment (start 26.04 4.6) (end 26.04 7.9) (width 0.8) (layer F.Cu) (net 24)))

